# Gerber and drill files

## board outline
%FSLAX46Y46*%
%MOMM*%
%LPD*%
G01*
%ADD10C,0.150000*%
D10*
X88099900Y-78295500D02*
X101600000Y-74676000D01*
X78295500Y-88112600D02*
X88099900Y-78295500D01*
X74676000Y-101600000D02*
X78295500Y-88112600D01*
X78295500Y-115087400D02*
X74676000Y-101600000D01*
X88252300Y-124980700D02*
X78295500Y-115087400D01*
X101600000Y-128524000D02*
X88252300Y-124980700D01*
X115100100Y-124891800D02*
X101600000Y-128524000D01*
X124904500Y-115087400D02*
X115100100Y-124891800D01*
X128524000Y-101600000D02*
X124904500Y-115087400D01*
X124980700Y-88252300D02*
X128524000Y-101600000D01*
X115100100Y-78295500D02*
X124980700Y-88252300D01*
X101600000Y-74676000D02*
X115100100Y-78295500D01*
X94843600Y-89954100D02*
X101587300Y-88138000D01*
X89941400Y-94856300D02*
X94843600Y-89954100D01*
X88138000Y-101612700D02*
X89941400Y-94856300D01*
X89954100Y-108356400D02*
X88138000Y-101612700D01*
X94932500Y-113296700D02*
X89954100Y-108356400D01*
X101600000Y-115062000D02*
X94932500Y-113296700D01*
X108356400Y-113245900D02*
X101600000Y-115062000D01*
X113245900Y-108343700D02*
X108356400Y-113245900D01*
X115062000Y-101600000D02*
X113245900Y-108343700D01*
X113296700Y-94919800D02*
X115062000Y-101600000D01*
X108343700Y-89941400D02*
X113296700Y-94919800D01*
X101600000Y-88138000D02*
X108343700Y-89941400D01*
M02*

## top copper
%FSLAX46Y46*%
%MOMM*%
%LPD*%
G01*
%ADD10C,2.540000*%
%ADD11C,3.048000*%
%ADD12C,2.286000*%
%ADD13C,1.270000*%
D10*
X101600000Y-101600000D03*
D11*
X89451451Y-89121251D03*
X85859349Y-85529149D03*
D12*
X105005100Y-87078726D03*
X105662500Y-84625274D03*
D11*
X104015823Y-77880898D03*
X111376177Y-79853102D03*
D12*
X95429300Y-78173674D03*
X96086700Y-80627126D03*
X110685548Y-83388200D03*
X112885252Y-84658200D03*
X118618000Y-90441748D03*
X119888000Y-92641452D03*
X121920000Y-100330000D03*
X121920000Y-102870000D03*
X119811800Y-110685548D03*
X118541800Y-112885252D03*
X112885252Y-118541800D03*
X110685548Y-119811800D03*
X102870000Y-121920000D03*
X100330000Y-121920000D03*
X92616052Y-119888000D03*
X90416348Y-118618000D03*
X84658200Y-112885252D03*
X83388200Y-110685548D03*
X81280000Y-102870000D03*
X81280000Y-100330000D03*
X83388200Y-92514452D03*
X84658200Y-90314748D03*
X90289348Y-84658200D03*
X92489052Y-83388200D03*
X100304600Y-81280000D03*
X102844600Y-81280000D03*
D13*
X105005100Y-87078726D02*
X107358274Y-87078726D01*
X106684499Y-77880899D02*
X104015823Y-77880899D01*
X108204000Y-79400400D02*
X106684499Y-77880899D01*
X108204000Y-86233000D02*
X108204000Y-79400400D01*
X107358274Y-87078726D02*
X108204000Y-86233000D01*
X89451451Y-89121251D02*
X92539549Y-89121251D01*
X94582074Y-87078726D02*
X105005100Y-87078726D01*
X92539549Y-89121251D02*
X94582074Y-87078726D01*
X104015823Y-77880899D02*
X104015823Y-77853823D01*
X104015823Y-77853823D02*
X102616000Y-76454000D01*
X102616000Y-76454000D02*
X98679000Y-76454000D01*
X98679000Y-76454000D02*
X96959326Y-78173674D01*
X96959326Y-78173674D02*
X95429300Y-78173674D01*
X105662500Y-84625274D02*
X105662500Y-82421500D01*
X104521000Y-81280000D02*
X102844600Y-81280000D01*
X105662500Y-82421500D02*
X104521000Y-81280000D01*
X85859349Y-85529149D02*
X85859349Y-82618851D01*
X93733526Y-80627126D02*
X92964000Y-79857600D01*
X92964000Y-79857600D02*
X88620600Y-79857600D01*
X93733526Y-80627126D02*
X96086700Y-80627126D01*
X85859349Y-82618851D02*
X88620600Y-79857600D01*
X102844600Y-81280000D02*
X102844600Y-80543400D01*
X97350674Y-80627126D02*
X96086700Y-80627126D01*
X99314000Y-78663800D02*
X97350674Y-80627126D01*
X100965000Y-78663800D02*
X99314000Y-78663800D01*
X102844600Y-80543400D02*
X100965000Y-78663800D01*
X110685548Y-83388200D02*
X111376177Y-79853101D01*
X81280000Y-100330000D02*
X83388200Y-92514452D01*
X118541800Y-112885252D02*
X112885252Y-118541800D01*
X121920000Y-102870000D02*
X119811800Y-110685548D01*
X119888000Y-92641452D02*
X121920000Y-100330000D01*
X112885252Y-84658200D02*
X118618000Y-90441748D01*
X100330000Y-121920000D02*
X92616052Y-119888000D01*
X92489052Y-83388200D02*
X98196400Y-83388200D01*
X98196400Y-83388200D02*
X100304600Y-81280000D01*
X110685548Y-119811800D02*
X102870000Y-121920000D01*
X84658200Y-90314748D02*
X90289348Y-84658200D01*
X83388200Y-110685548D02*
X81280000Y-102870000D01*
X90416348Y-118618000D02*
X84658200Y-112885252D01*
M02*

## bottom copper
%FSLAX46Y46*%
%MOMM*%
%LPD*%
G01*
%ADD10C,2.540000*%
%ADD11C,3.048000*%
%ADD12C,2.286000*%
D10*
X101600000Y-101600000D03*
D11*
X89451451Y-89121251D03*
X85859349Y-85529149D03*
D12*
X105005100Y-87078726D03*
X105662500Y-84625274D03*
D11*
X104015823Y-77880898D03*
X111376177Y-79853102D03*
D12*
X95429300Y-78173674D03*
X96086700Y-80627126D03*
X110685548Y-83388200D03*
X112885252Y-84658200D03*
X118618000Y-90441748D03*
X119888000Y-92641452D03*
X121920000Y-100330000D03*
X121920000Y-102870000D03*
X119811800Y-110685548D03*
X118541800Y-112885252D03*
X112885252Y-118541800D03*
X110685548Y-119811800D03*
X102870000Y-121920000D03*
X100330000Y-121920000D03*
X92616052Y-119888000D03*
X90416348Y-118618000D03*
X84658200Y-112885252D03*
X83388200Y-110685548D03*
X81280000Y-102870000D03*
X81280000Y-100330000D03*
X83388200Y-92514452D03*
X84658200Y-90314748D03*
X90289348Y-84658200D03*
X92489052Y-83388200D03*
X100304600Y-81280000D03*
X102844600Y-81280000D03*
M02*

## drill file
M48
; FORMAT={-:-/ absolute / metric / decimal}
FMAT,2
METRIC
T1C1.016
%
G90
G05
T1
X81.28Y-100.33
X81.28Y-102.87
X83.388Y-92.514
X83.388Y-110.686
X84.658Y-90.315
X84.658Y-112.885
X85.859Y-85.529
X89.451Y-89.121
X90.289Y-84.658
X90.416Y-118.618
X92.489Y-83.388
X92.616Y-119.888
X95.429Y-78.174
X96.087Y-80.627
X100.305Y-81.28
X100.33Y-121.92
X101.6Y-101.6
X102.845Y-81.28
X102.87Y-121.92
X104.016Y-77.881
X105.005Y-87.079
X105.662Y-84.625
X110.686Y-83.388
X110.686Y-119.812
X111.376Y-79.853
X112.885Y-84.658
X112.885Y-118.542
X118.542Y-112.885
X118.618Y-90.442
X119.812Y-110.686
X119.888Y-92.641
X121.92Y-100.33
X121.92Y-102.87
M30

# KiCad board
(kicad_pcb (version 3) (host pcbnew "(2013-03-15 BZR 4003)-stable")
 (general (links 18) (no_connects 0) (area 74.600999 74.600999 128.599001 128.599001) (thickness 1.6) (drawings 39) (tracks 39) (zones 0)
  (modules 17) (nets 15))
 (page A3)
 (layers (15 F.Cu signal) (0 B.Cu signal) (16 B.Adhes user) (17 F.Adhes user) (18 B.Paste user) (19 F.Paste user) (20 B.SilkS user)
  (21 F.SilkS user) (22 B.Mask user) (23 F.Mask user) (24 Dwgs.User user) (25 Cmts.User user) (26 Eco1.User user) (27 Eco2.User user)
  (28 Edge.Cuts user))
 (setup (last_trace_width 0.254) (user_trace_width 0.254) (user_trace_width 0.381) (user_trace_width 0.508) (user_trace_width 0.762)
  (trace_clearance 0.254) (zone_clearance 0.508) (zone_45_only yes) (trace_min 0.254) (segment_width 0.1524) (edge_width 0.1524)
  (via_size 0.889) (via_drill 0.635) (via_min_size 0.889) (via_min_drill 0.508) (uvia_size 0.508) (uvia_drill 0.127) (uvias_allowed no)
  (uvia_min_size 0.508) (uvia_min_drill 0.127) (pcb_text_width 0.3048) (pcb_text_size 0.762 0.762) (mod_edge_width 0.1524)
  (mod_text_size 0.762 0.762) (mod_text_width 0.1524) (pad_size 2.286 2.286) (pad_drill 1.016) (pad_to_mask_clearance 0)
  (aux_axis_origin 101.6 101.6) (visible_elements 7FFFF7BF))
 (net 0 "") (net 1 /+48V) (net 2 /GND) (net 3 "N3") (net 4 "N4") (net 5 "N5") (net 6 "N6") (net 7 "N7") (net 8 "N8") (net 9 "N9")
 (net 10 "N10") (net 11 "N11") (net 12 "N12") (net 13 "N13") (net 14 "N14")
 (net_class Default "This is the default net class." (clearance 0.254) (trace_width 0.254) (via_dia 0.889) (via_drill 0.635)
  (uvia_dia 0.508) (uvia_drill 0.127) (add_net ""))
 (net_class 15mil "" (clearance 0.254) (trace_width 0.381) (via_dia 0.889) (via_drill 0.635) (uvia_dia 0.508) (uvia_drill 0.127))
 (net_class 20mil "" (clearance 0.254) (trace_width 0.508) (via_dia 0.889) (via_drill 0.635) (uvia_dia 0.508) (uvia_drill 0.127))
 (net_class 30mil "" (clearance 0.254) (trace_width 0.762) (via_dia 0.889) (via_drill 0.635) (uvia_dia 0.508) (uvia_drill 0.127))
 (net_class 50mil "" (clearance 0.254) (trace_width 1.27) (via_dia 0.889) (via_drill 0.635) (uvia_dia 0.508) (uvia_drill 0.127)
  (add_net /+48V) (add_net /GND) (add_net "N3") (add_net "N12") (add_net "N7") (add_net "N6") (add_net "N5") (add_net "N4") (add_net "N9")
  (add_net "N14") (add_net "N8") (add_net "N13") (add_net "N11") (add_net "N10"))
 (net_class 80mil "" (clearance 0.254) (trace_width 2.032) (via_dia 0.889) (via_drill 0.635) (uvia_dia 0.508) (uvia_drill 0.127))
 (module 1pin (layer F.Cu) (at 101.6 101.6)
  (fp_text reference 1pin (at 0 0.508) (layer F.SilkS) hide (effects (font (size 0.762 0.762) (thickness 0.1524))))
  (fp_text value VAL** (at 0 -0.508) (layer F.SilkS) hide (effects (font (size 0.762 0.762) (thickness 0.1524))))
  (pad 1 thru_hole circle (at 0 0) (size 2.54 2.54) (drill 1.016) (layers *.Cu *.Mask F.SilkS)))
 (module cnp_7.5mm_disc (layer F.Cu) (at 87.6554 87.3252 135)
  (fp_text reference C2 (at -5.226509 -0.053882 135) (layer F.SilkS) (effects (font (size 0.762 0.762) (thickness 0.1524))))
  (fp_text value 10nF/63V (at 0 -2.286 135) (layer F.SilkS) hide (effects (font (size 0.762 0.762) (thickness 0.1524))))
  (pad 1 thru_hole circle (at -2.54 0 135) (size 3.048 3.048) (drill 1.016) (layers *.Cu *.Mask F.SilkS) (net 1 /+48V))
  (pad 2 thru_hole circle (at 2.54 0 135) (size 3.048 3.048) (drill 1.016) (layers *.Cu *.Mask F.SilkS) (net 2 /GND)))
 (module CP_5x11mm (layer F.Cu) (at 105.3338 85.852 345)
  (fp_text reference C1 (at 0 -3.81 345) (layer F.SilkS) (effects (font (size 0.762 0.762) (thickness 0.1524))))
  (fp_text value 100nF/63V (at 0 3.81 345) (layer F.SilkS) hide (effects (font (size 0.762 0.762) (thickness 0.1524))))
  (pad 1 thru_hole circle (at 0 1.27 345) (size 2.286 2.286) (drill 1.016) (layers *.Cu *.Mask F.SilkS) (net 1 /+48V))
  (pad 2 thru_hole circle (at 0 -1.27 345) (size 2.286 2.286) (drill 1.016) (layers *.Cu *.Mask F.SilkS) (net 2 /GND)))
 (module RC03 (layer F.Cu) (at 107.696 78.867 345) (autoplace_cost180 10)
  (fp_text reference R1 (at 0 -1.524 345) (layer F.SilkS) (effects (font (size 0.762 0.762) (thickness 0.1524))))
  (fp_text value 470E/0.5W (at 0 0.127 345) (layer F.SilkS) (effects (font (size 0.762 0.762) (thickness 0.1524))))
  (pad 1 thru_hole circle (at -3.81 -0.000001 345) (size 3.048 3.048) (drill 1.016) (layers *.Cu *.Mask F.SilkS) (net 1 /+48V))
  (pad 2 thru_hole circle (at 3.81 0.000001 345) (size 3.048 3.048) (drill 1.016) (layers *.Cu *.Mask F.SilkS) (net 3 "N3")))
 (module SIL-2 (layer F.Cu) (at 95.758 79.4004 285)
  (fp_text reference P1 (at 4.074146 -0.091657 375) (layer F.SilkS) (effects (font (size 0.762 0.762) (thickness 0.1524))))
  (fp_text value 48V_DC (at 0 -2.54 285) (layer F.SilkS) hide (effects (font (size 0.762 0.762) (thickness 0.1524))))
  (pad 1 thru_hole circle (at -1.27 0 285) (size 2.286 2.286) (drill 1.016) (layers *.Cu *.Mask F.SilkS) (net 1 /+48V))
  (pad 2 thru_hole circle (at 1.27 0 285) (size 2.286 2.286) (drill 1.016) (layers *.Cu *.Mask F.SilkS) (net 2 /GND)))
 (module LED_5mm (layer F.Cu) (at 111.7854 84.0232 330)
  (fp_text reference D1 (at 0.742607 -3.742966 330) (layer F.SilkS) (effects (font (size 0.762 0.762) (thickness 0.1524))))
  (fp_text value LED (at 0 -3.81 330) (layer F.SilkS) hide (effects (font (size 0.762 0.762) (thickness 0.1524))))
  (pad 1 thru_hole circle (at -1.27 0 330) (size 2.286 2.286) (drill 1.016) (layers *.Cu *.Mask F.SilkS) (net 3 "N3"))
  (pad 2 thru_hole circle (at 1.27 0 330) (size 2.286 2.286) (drill 1.016) (layers *.Cu *.Mask F.SilkS) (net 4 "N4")))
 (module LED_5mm (layer F.Cu) (at 119.253 91.5416 300)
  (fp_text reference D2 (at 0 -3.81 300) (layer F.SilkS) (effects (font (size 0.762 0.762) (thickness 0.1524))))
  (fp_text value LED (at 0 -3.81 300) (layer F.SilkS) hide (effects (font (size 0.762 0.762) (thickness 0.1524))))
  (pad 1 thru_hole circle (at -1.27 0 300) (size 2.286 2.286) (drill 1.016) (layers *.Cu *.Mask F.SilkS) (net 4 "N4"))
  (pad 2 thru_hole circle (at 1.27 0 300) (size 2.286 2.286) (drill 1.016) (layers *.Cu *.Mask F.SilkS) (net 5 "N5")))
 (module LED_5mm (layer F.Cu) (at 121.92 101.6 270)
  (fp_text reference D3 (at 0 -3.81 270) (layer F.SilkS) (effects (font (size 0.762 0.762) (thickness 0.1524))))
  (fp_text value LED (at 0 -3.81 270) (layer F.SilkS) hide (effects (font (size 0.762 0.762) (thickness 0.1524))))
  (pad 1 thru_hole circle (at -1.27 0 270) (size 2.286 2.286) (drill 1.016) (layers *.Cu *.Mask F.SilkS) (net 5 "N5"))
  (pad 2 thru_hole circle (at 1.27 0 270) (size 2.286 2.286) (drill 1.016) (layers *.Cu *.Mask F.SilkS) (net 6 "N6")))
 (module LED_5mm (layer F.Cu) (at 119.1768 111.7854 240)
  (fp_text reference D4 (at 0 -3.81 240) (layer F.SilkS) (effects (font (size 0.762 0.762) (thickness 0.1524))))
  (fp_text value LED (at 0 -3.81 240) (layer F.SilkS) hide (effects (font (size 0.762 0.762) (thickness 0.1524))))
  (pad 1 thru_hole circle (at -1.27 0 240) (size 2.286 2.286) (drill 1.016) (layers *.Cu *.Mask F.SilkS) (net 6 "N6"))
  (pad 2 thru_hole circle (at 1.27 0 240) (size 2.286 2.286) (drill 1.016) (layers *.Cu *.Mask F.SilkS) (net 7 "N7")))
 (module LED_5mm (layer F.Cu) (at 111.7854 119.1768 210)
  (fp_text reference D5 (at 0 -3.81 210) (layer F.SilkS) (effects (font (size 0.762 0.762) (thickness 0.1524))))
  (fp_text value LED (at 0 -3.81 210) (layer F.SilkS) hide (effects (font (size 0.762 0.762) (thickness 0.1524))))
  (pad 1 thru_hole circle (at -1.27 0 210) (size 2.286 2.286) (drill 1.016) (layers *.Cu *.Mask F.SilkS) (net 7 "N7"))
  (pad 2 thru_hole circle (at 1.27 0 210) (size 2.286 2.286) (drill 1.016) (layers *.Cu *.Mask F.SilkS) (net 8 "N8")))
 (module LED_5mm (layer F.Cu) (at 101.6 121.92 180)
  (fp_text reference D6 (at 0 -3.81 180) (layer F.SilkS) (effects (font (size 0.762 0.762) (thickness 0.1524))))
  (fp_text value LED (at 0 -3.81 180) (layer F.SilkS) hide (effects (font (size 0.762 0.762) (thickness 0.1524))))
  (pad 1 thru_hole circle (at -1.27 0 180) (size 2.286 2.286) (drill 1.016) (layers *.Cu *.Mask F.SilkS) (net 8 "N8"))
  (pad 2 thru_hole circle (at 1.27 0 180) (size 2.286 2.286) (drill 1.016) (layers *.Cu *.Mask F.SilkS) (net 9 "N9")))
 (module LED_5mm (layer F.Cu) (at 91.5162 119.253 150)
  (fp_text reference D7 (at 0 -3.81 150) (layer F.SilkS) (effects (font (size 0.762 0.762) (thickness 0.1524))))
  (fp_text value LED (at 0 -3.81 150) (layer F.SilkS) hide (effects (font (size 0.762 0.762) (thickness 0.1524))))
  (pad 1 thru_hole circle (at -1.27 0 150) (size 2.286 2.286) (drill 1.016) (layers *.Cu *.Mask F.SilkS) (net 9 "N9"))
  (pad 2 thru_hole circle (at 1.27 0 150) (size 2.286 2.286) (drill 1.016) (layers *.Cu *.Mask F.SilkS) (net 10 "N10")))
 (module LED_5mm (layer F.Cu) (at 84.0232 111.7854 120)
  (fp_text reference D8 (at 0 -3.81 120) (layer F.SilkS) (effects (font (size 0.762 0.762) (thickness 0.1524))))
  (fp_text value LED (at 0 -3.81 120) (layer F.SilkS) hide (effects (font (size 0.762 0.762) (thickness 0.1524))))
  (pad 1 thru_hole circle (at -1.27 0 120) (size 2.286 2.286) (drill 1.016) (layers *.Cu *.Mask F.SilkS) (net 10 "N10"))
  (pad 2 thru_hole circle (at 1.27 0 120) (size 2.286 2.286) (drill 1.016) (layers *.Cu *.Mask F.SilkS) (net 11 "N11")))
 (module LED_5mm (layer F.Cu) (at 81.28 101.6 90)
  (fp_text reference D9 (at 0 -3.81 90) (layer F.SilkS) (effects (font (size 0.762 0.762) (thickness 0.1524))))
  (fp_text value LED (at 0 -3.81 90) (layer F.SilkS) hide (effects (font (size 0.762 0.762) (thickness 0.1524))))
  (pad 1 thru_hole circle (at -1.27 0 90) (size 2.286 2.286) (drill 1.016) (layers *.Cu *.Mask F.SilkS) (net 11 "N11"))
  (pad 2 thru_hole circle (at 1.27 0 90) (size 2.286 2.286) (drill 1.016) (layers *.Cu *.Mask F.SilkS) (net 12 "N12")))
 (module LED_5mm (layer F.Cu) (at 84.0232 91.4146 60)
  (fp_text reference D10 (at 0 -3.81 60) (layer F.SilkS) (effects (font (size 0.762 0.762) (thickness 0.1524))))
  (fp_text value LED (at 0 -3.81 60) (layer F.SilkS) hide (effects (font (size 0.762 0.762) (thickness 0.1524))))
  (pad 1 thru_hole circle (at -1.27 0 60) (size 2.286 2.286) (drill 1.016) (layers *.Cu *.Mask F.SilkS) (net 12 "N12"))
  (pad 2 thru_hole circle (at 1.27 0 60) (size 2.286 2.286) (drill 1.016) (layers *.Cu *.Mask F.SilkS) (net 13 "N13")))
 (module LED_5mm (layer F.Cu) (at 91.3892 84.0232 30)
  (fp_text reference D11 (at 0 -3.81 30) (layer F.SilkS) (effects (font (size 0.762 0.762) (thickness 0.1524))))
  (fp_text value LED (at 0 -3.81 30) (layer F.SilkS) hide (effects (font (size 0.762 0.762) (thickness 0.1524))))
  (pad 1 thru_hole circle (at -1.27 0 30) (size 2.286 2.286) (drill 1.016) (layers *.Cu *.Mask F.SilkS) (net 13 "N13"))
  (pad 2 thru_hole circle (at 1.27 0 30) (size 2.286 2.286) (drill 1.016) (layers *.Cu *.Mask F.SilkS) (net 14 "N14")))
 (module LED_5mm (layer F.Cu) (at 101.5746 81.28)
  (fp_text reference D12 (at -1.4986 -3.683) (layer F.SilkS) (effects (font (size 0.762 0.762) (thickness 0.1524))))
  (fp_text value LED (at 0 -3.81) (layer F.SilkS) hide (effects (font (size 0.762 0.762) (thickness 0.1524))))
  (pad 1 thru_hole circle (at -1.27 0) (size 2.286 2.286) (drill 1.016) (layers *.Cu *.Mask F.SilkS) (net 14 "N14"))
  (pad 2 thru_hole circle (at 1.27 0) (size 2.286 2.286) (drill 1.016) (layers *.Cu *.Mask F.SilkS) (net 2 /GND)))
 (gr_line (start 88.0999 78.2955) (end 101.6 74.676) (angle 90) (layer Edge.Cuts) (width 0.15))
 (gr_line (start 78.2955 88.1126) (end 88.0999 78.2955) (angle 90) (layer Edge.Cuts) (width 0.15))
 (gr_line (start 74.676 101.6) (end 78.2955 88.1126) (angle 90) (layer Edge.Cuts) (width 0.15))
 (gr_line (start 78.2955 115.0874) (end 74.676 101.6) (angle 90) (layer Edge.Cuts) (width 0.15))
 (gr_line (start 88.2523 124.9807) (end 78.2955 115.0874) (angle 90) (layer Edge.Cuts) (width 0.15))
 (gr_line (start 101.6 128.524) (end 88.2523 124.9807) (angle 90) (layer Edge.Cuts) (width 0.15))
 (gr_line (start 115.1001 124.8918) (end 101.6 128.524) (angle 90) (layer Edge.Cuts) (width 0.15))
 (gr_line (start 124.9045 115.0874) (end 115.1001 124.8918) (angle 90) (layer Edge.Cuts) (width 0.15))
 (gr_line (start 128.524 101.6) (end 124.9045 115.0874) (angle 90) (layer Edge.Cuts) (width 0.15))
 (gr_line (start 124.9807 88.2523) (end 128.524 101.6) (angle 90) (layer Edge.Cuts) (width 0.15))
 (gr_line (start 115.1001 78.2955) (end 124.9807 88.2523) (angle 90) (layer Edge.Cuts) (width 0.15))
 (gr_line (start 101.6 74.676) (end 115.1001 78.2955) (angle 90) (layer Edge.Cuts) (width 0.15))
 (gr_line (start 94.8436 89.9541) (end 101.5873 88.138) (angle 90) (layer Edge.Cuts) (width 0.15))
 (gr_line (start 89.9414 94.8563) (end 94.8436 89.9541) (angle 90) (layer Edge.Cuts) (width 0.15))
 (gr_line (start 88.138 101.6127) (end 89.9414 94.8563) (angle 90) (layer Edge.Cuts) (width 0.15))
 (gr_line (start 89.9541 108.3564) (end 88.138 101.6127) (angle 90) (layer Edge.Cuts) (width 0.15))
 (gr_line (start 94.9325 113.2967) (end 89.9541 108.3564) (angle 90) (layer Edge.Cuts) (width 0.15))
 (gr_line (start 101.6 115.062) (end 94.9325 113.2967) (angle 90) (layer Edge.Cuts) (width 0.15))
 (gr_line (start 108.3564 113.2459) (end 101.6 115.062) (angle 90) (layer Edge.Cuts) (width 0.15))
 (gr_line (start 113.2459 108.3437) (end 108.3564 113.2459) (angle 90) (layer Edge.Cuts) (width 0.15))
 (gr_line (start 115.062 101.6) (end 113.2459 108.3437) (angle 90) (layer Edge.Cuts) (width 0.15))
 (gr_line (start 113.2967 94.9198) (end 115.062 101.6) (angle 90) (layer Edge.Cuts) (width 0.15))
 (gr_line (start 108.3437 89.9414) (end 113.2967 94.9198) (angle 90) (layer Edge.Cuts) (width 0.15))
 (gr_line (start 101.6 88.138) (end 108.3437 89.9414) (angle 90) (layer Edge.Cuts) (width 0.15))
 (segment (start 105.0051 87.078726) (end 107.358274 87.078726) (width 1.27) (layer F.Cu) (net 1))
 (segment (start 106.684499 77.880899) (end 104.015823 77.880899) (width 1.27) (layer F.Cu) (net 1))
 (segment (start 108.204 79.4004) (end 106.684499 77.880899) (width 1.27) (layer F.Cu) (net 1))
 (segment (start 108.204 86.233) (end 108.204 79.4004) (width 1.27) (layer F.Cu) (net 1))
 (segment (start 107.358274 87.078726) (end 108.204 86.233) (width 1.27) (layer F.Cu) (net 1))
 (segment (start 89.451451 89.121251) (end 92.539549 89.121251) (width 1.27) (layer F.Cu) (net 1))
 (segment (start 94.582074 87.078726) (end 105.0051 87.078726) (width 1.27) (layer F.Cu) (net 1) (status 20))
 (segment (start 92.539549 89.121251) (end 94.582074 87.078726) (width 1.27) (layer F.Cu) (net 1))
 (segment (start 104.015823 77.880899) (end 104.015823 77.853823) (width 1.27) (layer F.Cu) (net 1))
 (segment (start 104.015823 77.853823) (end 102.616 76.454) (width 1.27) (layer F.Cu) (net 1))
 (segment (start 102.616 76.454) (end 98.679 76.454) (width 1.27) (layer F.Cu) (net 1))
 (segment (start 98.679 76.454) (end 96.959326 78.173674) (width 1.27) (layer F.Cu) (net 1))
 (segment (start 96.959326 78.173674) (end 95.4293 78.173674) (width 1.27) (layer F.Cu) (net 1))
 (segment (start 105.6625 84.625274) (end 105.6625 82.4215) (width 1.27) (layer F.Cu) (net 2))
 (segment (start 104.521 81.28) (end 102.8446 81.28) (width 1.27) (layer F.Cu) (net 2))
 (segment (start 105.6625 82.4215) (end 104.521 81.28) (width 1.27) (layer F.Cu) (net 2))
 (segment (start 85.859349 85.529149) (end 85.859349 82.618851) (width 1.27) (layer F.Cu) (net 2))
 (segment (start 93.733526 80.627126) (end 92.964 79.8576) (width 1.27) (layer F.Cu) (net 2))
 (segment (start 92.964 79.8576) (end 88.6206 79.8576) (width 1.27) (layer F.Cu) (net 2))
 (segment (start 93.733526 80.627126) (end 96.0867 80.627126) (width 1.27) (layer F.Cu) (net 2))
 (segment (start 85.859349 82.618851) (end 88.6206 79.8576) (width 1.27) (layer F.Cu) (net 2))
 (segment (start 102.8446 81.28) (end 102.8446 80.5434) (width 1.27) (layer F.Cu) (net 2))
 (segment (start 97.350674 80.627126) (end 96.0867 80.627126) (width 1.27) (layer F.Cu) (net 2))
 (segment (start 99.314 78.6638) (end 97.350674 80.627126) (width 1.27) (layer F.Cu) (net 2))
 (segment (start 100.965 78.6638) (end 99.314 78.6638) (width 1.27) (layer F.Cu) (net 2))
 (segment (start 102.8446 80.5434) (end 100.965 78.6638) (width 1.27) (layer F.Cu) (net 2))
 (segment (start 110.685548 83.3882) (end 111.376177 79.853101) (width 1.27) (layer F.Cu) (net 3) (status 30))
 (segment (start 81.28 100.33) (end 83.3882 92.514452) (width 1.27) (layer F.Cu) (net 12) (status 30))
 (segment (start 118.5418 112.885252) (end 112.885252 118.5418) (width 1.27) (layer F.Cu) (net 7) (status 30))
 (segment (start 121.92 102.87) (end 119.8118 110.685548) (width 1.27) (layer F.Cu) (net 6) (status 30))
 (segment (start 119.888 92.641452) (end 121.92 100.33) (width 1.27) (layer F.Cu) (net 5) (status 30))
 (segment (start 112.885252 84.6582) (end 118.618 90.441748) (width 1.27) (layer F.Cu) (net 4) (status 30))
 (segment (start 100.33 121.92) (end 92.616052 119.888) (width 1.27) (layer F.Cu) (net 9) (status 30))
 (segment (start 92.489052 83.3882) (end 98.1964 83.3882) (width 1.27) (layer F.Cu) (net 14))
 (segment (start 98.1964 83.3882) (end 100.3046 81.28) (width 1.27) (layer F.Cu) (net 14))
 (segment (start 110.685548 119.8118) (end 102.87 121.92) (width 1.27) (layer F.Cu) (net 8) (status 30))
 (segment (start 84.6582 90.314748) (end 90.289348 84.6582) (width 1.27) (layer F.Cu) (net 13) (status 30))
 (segment (start 83.3882 110.685548) (end 81.28 102.87) (width 1.27) (layer F.Cu) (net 11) (status 30))
 (segment (start 90.416348 118.618) (end 84.6582 112.885252) (width 1.27) (layer F.Cu) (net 10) (status 30)))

